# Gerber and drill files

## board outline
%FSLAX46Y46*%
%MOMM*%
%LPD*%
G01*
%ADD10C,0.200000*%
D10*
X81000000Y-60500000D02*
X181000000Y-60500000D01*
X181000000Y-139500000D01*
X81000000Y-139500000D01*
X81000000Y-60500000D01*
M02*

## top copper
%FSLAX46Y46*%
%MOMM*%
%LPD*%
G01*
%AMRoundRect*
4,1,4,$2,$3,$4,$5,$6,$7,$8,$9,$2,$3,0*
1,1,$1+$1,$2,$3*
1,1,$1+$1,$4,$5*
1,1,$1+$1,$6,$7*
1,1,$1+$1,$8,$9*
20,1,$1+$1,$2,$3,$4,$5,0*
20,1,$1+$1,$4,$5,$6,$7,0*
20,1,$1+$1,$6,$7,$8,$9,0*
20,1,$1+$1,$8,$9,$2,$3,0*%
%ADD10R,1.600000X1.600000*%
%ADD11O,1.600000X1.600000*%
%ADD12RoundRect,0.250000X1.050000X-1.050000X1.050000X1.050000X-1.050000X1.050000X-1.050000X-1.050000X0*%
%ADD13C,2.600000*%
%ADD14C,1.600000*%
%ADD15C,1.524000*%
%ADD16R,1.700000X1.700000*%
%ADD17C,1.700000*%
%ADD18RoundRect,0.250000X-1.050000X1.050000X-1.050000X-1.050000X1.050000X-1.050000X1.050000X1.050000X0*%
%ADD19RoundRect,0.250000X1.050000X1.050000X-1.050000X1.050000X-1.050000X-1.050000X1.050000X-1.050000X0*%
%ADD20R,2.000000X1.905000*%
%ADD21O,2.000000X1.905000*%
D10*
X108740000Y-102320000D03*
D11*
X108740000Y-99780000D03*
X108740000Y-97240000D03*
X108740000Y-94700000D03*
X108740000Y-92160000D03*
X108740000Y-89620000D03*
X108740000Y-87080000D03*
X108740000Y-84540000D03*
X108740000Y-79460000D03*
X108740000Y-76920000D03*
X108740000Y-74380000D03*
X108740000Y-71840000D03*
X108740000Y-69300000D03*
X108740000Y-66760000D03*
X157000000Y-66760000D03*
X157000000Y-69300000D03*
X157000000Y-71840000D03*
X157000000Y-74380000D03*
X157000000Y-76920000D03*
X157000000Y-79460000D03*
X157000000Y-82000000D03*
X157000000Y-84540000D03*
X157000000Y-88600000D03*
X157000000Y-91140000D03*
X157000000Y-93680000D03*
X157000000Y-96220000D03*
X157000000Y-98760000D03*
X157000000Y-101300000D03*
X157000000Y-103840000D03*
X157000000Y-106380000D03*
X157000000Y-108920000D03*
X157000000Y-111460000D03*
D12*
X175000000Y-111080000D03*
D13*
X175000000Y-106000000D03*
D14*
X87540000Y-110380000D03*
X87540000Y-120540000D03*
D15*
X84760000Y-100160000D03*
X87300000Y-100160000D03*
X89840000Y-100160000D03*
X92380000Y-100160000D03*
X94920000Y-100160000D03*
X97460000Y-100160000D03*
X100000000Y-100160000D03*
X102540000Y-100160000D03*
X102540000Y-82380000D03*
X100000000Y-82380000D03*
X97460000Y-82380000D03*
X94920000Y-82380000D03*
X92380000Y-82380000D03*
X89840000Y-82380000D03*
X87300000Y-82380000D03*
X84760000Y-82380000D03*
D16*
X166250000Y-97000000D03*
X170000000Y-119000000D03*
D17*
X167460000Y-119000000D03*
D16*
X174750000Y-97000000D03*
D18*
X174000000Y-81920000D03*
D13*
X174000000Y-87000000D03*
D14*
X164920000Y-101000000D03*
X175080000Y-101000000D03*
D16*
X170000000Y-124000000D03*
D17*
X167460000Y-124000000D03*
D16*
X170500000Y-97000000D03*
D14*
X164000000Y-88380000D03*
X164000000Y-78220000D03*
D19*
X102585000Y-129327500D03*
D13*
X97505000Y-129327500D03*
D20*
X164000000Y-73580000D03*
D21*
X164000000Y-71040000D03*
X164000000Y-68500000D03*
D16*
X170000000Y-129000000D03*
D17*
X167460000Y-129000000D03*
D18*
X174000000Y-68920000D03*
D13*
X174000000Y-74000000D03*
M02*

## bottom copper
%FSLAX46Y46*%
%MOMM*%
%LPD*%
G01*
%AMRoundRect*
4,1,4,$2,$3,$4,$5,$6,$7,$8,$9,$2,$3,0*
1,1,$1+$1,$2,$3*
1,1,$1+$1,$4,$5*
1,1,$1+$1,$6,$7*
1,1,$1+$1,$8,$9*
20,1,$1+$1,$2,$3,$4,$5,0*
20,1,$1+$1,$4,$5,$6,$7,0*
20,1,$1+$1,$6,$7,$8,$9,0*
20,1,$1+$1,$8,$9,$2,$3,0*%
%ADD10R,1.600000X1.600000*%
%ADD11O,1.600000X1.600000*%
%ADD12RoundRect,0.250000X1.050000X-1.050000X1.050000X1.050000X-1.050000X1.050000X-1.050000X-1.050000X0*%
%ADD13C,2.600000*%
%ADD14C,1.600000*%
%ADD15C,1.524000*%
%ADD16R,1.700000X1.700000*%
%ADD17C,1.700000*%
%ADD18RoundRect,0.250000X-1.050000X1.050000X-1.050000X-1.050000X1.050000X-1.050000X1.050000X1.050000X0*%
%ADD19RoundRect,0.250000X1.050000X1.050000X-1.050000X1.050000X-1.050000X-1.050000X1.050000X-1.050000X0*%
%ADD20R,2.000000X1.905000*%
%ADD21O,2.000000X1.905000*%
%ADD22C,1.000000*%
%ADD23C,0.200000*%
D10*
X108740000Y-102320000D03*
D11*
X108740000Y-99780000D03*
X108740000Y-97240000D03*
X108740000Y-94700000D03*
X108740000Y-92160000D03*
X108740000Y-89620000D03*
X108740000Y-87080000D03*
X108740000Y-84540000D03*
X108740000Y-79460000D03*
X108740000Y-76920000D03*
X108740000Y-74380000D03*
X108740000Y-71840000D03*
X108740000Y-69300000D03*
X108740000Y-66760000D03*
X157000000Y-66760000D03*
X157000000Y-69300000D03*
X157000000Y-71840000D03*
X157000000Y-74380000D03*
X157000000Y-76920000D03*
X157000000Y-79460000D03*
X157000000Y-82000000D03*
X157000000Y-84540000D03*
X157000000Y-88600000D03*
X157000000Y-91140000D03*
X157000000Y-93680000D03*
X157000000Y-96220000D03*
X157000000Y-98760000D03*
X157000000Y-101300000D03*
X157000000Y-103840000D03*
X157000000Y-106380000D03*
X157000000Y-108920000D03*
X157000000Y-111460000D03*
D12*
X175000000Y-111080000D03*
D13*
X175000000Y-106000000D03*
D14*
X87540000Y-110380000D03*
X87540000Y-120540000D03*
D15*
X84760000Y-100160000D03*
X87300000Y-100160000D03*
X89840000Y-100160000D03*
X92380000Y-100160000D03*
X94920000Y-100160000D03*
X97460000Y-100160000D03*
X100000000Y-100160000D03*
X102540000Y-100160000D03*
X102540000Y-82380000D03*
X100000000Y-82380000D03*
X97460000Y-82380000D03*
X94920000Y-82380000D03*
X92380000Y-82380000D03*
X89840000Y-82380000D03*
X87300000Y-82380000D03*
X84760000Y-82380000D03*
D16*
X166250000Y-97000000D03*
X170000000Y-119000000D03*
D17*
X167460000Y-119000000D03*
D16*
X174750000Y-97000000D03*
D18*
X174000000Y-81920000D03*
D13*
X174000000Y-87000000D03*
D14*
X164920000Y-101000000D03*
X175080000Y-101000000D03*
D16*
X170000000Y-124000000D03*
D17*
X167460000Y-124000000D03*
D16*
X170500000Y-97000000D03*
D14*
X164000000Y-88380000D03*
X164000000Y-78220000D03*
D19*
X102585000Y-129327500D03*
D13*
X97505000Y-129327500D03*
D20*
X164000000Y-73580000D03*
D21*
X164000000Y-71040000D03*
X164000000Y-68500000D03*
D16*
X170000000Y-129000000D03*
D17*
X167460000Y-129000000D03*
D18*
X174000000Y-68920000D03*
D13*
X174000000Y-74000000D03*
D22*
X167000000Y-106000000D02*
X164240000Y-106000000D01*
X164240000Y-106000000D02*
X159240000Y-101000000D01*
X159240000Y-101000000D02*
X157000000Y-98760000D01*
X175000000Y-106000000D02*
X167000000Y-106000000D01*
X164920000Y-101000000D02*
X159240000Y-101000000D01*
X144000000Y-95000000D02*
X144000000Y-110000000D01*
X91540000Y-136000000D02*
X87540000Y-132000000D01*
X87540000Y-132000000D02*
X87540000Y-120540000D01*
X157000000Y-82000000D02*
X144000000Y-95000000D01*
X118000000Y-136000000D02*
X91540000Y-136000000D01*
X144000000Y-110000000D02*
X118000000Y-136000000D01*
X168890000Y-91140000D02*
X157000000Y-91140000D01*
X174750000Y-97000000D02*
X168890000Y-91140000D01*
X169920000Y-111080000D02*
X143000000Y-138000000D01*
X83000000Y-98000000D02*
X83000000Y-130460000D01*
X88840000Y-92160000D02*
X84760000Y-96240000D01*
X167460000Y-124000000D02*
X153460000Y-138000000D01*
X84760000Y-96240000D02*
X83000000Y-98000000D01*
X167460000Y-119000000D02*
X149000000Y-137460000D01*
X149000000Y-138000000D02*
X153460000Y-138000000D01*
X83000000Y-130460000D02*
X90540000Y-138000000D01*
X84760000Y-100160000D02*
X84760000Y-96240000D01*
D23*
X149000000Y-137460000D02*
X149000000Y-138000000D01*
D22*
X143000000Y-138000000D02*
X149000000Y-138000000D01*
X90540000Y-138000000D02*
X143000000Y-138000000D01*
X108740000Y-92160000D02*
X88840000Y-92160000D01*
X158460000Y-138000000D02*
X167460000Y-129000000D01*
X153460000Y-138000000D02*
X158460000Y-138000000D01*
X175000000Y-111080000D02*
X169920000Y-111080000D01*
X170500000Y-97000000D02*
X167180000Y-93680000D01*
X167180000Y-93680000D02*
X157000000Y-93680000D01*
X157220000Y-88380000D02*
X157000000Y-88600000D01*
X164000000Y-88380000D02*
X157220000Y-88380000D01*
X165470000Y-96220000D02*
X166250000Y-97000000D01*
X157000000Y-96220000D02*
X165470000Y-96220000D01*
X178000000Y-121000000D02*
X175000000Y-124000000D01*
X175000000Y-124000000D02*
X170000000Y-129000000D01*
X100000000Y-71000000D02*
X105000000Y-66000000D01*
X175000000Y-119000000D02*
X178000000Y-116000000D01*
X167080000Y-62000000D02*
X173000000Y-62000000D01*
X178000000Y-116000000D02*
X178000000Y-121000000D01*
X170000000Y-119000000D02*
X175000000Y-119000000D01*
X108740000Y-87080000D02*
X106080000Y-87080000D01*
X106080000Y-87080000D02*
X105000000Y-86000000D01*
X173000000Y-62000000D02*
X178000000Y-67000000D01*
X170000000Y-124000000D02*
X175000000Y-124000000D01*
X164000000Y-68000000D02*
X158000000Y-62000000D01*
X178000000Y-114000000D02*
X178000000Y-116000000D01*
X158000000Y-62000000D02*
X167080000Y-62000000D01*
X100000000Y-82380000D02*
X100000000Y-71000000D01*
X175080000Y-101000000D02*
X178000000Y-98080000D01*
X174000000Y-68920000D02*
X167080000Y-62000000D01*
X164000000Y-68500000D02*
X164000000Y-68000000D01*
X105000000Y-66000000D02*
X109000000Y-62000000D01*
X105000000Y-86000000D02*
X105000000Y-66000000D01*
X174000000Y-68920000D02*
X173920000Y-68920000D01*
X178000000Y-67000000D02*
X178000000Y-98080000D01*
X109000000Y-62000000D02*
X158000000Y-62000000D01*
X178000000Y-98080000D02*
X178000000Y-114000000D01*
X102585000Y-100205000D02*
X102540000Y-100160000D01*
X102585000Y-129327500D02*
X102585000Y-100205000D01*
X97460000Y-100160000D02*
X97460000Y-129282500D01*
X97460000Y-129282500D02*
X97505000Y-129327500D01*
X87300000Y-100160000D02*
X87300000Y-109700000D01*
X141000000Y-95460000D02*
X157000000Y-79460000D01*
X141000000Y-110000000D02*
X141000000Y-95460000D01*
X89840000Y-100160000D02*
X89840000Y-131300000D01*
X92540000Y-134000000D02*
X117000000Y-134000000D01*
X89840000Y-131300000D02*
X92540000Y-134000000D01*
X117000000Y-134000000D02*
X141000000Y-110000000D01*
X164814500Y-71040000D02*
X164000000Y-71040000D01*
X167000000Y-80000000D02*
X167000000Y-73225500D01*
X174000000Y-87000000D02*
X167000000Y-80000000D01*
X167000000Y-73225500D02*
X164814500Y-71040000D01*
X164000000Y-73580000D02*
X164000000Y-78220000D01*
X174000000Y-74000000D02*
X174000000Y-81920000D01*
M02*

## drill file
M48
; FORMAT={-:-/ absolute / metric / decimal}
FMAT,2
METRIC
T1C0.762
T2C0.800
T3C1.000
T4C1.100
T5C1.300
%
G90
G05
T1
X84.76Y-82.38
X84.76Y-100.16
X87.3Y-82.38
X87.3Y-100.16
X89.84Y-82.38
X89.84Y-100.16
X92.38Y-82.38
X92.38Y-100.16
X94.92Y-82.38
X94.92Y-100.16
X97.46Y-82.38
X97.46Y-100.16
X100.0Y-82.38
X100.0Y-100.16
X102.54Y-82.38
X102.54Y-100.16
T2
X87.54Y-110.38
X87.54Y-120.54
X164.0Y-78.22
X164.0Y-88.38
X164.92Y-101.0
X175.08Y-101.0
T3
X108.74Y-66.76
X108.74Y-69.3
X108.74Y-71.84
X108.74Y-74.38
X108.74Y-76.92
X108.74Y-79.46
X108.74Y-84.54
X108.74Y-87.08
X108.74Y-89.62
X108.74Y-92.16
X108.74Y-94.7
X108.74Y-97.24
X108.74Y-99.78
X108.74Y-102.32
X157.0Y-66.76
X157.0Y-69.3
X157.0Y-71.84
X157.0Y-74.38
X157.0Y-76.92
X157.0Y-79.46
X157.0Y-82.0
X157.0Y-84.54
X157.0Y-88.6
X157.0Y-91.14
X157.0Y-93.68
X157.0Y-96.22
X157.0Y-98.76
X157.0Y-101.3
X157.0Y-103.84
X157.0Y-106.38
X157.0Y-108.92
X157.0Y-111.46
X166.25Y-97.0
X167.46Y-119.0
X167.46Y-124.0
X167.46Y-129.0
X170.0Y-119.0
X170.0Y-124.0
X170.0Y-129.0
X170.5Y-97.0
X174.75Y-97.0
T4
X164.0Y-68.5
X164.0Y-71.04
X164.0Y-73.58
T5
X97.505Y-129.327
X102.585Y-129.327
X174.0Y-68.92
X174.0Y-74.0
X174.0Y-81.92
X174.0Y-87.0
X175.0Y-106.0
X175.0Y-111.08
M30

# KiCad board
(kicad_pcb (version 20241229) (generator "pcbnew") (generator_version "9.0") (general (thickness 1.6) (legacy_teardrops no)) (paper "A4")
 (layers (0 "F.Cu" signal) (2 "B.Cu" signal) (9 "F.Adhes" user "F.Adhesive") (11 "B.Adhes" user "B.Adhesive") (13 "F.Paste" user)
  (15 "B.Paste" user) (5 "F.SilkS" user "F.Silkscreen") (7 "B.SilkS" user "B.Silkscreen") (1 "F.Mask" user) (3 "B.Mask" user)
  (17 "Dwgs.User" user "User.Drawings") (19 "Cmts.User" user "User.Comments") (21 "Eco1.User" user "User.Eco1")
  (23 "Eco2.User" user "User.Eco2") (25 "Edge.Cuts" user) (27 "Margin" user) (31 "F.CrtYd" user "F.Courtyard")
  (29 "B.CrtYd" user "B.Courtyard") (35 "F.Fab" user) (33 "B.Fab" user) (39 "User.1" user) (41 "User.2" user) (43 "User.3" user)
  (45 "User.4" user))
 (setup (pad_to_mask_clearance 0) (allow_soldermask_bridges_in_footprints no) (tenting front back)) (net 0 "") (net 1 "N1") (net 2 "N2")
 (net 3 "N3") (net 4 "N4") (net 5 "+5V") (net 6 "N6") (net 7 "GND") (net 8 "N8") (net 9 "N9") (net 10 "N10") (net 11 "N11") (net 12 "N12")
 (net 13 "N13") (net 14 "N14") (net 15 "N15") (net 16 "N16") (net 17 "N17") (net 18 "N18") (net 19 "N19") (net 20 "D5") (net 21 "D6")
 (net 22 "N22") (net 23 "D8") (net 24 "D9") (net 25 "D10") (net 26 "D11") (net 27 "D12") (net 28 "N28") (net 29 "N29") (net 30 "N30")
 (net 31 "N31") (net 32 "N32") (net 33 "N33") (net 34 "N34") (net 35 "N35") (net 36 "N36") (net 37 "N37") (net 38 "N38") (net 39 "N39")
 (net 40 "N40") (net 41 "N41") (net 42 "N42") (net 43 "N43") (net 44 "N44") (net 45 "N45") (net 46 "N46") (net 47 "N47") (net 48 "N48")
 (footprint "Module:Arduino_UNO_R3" (layer "F.Cu") (at 108.74 102.32 90)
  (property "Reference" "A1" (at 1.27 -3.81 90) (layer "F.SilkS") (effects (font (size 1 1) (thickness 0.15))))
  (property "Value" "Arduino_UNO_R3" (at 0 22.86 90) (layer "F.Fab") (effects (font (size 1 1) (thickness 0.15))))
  (pad "1" thru_hole rect (at 0 0 180) (size 1.6 1.6) (drill 1) (layers "*.Cu" "*.Mask") (remove_unused_layers no) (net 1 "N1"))
  (pad "2" thru_hole oval (at 2.54 0 180) (size 1.6 1.6) (drill 1) (layers "*.Cu" "*.Mask") (remove_unused_layers no) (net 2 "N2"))
  (pad "3" thru_hole oval (at 5.08 0 180) (size 1.6 1.6) (drill 1) (layers "*.Cu" "*.Mask") (remove_unused_layers no) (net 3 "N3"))
  (pad "4" thru_hole oval (at 7.62 0 180) (size 1.6 1.6) (drill 1) (layers "*.Cu" "*.Mask") (remove_unused_layers no) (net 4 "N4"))
  (pad "5" thru_hole oval (at 10.16 0 180) (size 1.6 1.6) (drill 1) (layers "*.Cu" "*.Mask") (remove_unused_layers no) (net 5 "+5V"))
  (pad "6" thru_hole oval (at 12.7 0 180) (size 1.6 1.6) (drill 1) (layers "*.Cu" "*.Mask") (remove_unused_layers no) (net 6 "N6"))
  (pad "7" thru_hole oval (at 15.24 0 180) (size 1.6 1.6) (drill 1) (layers "*.Cu" "*.Mask") (remove_unused_layers no) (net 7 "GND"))
  (pad "8" thru_hole oval (at 17.78 0 180) (size 1.6 1.6) (drill 1) (layers "*.Cu" "*.Mask") (remove_unused_layers no) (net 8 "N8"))
  (pad "9" thru_hole oval (at 22.86 0 180) (size 1.6 1.6) (drill 1) (layers "*.Cu" "*.Mask") (remove_unused_layers no) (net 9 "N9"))
  (pad "10" thru_hole oval (at 25.4 0 180) (size 1.6 1.6) (drill 1) (layers "*.Cu" "*.Mask") (remove_unused_layers no) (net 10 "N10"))
  (pad "11" thru_hole oval (at 27.94 0 180) (size 1.6 1.6) (drill 1) (layers "*.Cu" "*.Mask") (remove_unused_layers no) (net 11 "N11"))
  (pad "12" thru_hole oval (at 30.48 0 180) (size 1.6 1.6) (drill 1) (layers "*.Cu" "*.Mask") (remove_unused_layers no) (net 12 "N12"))
  (pad "13" thru_hole oval (at 33.02 0 180) (size 1.6 1.6) (drill 1) (layers "*.Cu" "*.Mask") (remove_unused_layers no) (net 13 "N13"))
  (pad "14" thru_hole oval (at 35.56 0 180) (size 1.6 1.6) (drill 1) (layers "*.Cu" "*.Mask") (remove_unused_layers no) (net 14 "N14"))
  (pad "15" thru_hole oval (at 35.56 48.26 180) (size 1.6 1.6) (drill 1) (layers "*.Cu" "*.Mask") (remove_unused_layers no) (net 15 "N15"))
  (pad "16" thru_hole oval (at 33.02 48.26 180) (size 1.6 1.6) (drill 1) (layers "*.Cu" "*.Mask") (remove_unused_layers no) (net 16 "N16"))
  (pad "17" thru_hole oval (at 30.48 48.26 180) (size 1.6 1.6) (drill 1) (layers "*.Cu" "*.Mask") (remove_unused_layers no) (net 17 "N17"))
  (pad "18" thru_hole oval (at 27.94 48.26 180) (size 1.6 1.6) (drill 1) (layers "*.Cu" "*.Mask") (remove_unused_layers no) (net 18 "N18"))
  (pad "19" thru_hole oval (at 25.4 48.26 180) (size 1.6 1.6) (drill 1) (layers "*.Cu" "*.Mask") (remove_unused_layers no) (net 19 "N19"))
  (pad "20" thru_hole oval (at 22.86 48.26 180) (size 1.6 1.6) (drill 1) (layers "*.Cu" "*.Mask") (remove_unused_layers no) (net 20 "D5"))
  (pad "21" thru_hole oval (at 20.32 48.26 180) (size 1.6 1.6) (drill 1) (layers "*.Cu" "*.Mask") (remove_unused_layers no) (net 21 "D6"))
  (pad "22" thru_hole oval (at 17.78 48.26 180) (size 1.6 1.6) (drill 1) (layers "*.Cu" "*.Mask") (remove_unused_layers no) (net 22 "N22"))
  (pad "23" thru_hole oval (at 13.72 48.26 180) (size 1.6 1.6) (drill 1) (layers "*.Cu" "*.Mask") (remove_unused_layers no) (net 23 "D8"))
  (pad "24" thru_hole oval (at 11.18 48.26 180) (size 1.6 1.6) (drill 1) (layers "*.Cu" "*.Mask") (remove_unused_layers no) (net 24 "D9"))
  (pad "25" thru_hole oval (at 8.64 48.26 180) (size 1.6 1.6) (drill 1) (layers "*.Cu" "*.Mask") (remove_unused_layers no) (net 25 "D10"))
  (pad "26" thru_hole oval (at 6.1 48.26 180) (size 1.6 1.6) (drill 1) (layers "*.Cu" "*.Mask") (remove_unused_layers no) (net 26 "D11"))
  (pad "27" thru_hole oval (at 3.56 48.26 180) (size 1.6 1.6) (drill 1) (layers "*.Cu" "*.Mask") (remove_unused_layers no) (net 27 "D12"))
  (pad "28" thru_hole oval (at 1.02 48.26 180) (size 1.6 1.6) (drill 1) (layers "*.Cu" "*.Mask") (remove_unused_layers no) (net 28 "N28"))
  (pad "29" thru_hole oval (at -1.52 48.26 180) (size 1.6 1.6) (drill 1) (layers "*.Cu" "*.Mask") (remove_unused_layers no) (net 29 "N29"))
  (pad "30" thru_hole oval (at -4.06 48.26 180) (size 1.6 1.6) (drill 1) (layers "*.Cu" "*.Mask") (remove_unused_layers no) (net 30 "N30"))
  (pad "31" thru_hole oval (at -6.6 48.26 180) (size 1.6 1.6) (drill 1) (layers "*.Cu" "*.Mask") (remove_unused_layers no) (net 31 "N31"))
  (pad "32" thru_hole oval (at -9.14 48.26 180) (size 1.6 1.6) (drill 1) (layers "*.Cu" "*.Mask") (remove_unused_layers no) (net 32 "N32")))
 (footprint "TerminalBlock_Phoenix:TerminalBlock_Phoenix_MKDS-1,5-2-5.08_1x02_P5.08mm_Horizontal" (layer "F.Cu") (at 175 111.08 90)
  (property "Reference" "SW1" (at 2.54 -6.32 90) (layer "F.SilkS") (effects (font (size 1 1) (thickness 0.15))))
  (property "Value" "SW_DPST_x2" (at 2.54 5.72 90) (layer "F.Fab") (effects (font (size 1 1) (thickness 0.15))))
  (pad "1" thru_hole roundrect (at 0 0 90) (size 2.6 2.6) (drill 1.3) (layers "*.Cu" "*.Mask") (remove_unused_layers no)
   (roundrect_rratio 0.096154) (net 5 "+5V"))
  (pad "2" thru_hole circle (at 5.08 0 90) (size 2.6 2.6) (drill 1.3) (layers "*.Cu" "*.Mask") (remove_unused_layers no) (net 27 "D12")))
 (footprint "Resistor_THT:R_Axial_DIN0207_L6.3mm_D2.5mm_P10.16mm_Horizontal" (layer "F.Cu") (at 87.54 110.38 -90)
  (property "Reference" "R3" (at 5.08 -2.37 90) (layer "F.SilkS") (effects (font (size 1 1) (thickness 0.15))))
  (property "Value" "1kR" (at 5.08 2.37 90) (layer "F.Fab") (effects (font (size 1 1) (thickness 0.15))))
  (pad "1" thru_hole circle (at 0 0 270) (size 1.6 1.6) (drill 0.8) (layers "*.Cu" "*.Mask") (remove_unused_layers no) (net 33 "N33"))
  (pad "2" thru_hole circle (at 10.16 0 270) (size 1.6 1.6) (drill 0.8) (layers "*.Cu" "*.Mask") (remove_unused_layers no) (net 21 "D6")))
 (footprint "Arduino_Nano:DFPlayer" (layer "F.Cu") (at 84.76 92.54 90)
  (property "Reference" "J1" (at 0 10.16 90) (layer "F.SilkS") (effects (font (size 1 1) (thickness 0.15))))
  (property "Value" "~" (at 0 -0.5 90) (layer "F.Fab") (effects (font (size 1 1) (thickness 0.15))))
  (pad "1" thru_hole circle (at -7.62 0 90) (size 1.524 1.524) (drill 0.762) (layers "*.Cu" "*.Mask") (remove_unused_layers no)
   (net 5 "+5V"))
  (pad "2" thru_hole circle (at -7.62 2.54 90) (size 1.524 1.524) (drill 0.762) (layers "*.Cu" "*.Mask") (remove_unused_layers no)
   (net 33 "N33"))
  (pad "3" thru_hole circle (at -7.62 5.08 90) (size 1.524 1.524) (drill 0.762) (layers "*.Cu" "*.Mask") (remove_unused_layers no)
   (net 20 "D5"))
  (pad "4" thru_hole circle (at -7.62 7.62 90) (size 1.524 1.524) (drill 0.762) (layers "*.Cu" "*.Mask") (remove_unused_layers no)
   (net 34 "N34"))
  (pad "5" thru_hole circle (at -7.62 10.16 90) (size 1.524 1.524) (drill 0.762) (layers "*.Cu" "*.Mask") (remove_unused_layers no)
   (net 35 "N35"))
  (pad "6" thru_hole circle (at -7.62 12.7 90) (size 1.524 1.524) (drill 0.762) (layers "*.Cu" "*.Mask") (remove_unused_layers no)
   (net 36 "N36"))
  (pad "7" thru_hole circle (at -7.62 15.24 90) (size 1.524 1.524) (drill 0.762) (layers "*.Cu" "*.Mask") (remove_unused_layers no)
   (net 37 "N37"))
  (pad "8" thru_hole circle (at -7.62 17.78 90) (size 1.524 1.524) (drill 0.762) (layers "*.Cu" "*.Mask") (remove_unused_layers no)
   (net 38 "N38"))
  (pad "9" thru_hole circle (at 10.16 17.78 90) (size 1.524 1.524) (drill 0.762) (layers "*.Cu" "*.Mask") (remove_unused_layers no)
   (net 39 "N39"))
  (pad "10" thru_hole circle (at 10.16 15.24 90) (size 1.524 1.524) (drill 0.762) (layers "*.Cu" "*.Mask") (remove_unused_layers no)
   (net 7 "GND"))
  (pad "11" thru_hole circle (at 10.16 12.7 90) (size 1.524 1.524) (drill 0.762) (layers "*.Cu" "*.Mask") (remove_unused_layers no)
   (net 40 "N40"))
  (pad "12" thru_hole circle (at 10.16 10.16 90) (size 1.524 1.524) (drill 0.762) (layers "*.Cu" "*.Mask") (remove_unused_layers no)
   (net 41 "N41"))
  (pad "13" thru_hole circle (at 10.16 7.62 90) (size 1.524 1.524) (drill 0.762) (layers "*.Cu" "*.Mask") (remove_unused_layers no)
   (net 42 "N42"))
  (pad "14" thru_hole circle (at 10.16 5.08 90) (size 1.524 1.524) (drill 0.762) (layers "*.Cu" "*.Mask") (remove_unused_layers no)
   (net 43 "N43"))
  (pad "15" thru_hole circle (at 10.16 2.54 90) (size 1.524 1.524) (drill 0.762) (layers "*.Cu" "*.Mask") (remove_unused_layers no)
   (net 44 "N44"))
  (pad "16" thru_hole circle (at 10.16 0 90) (size 1.524 1.524) (drill 0.762) (layers "*.Cu" "*.Mask") (remove_unused_layers no)
   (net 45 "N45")))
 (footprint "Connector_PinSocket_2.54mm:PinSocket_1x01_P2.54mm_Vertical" (layer "F.Cu") (at 166.25 97 -90)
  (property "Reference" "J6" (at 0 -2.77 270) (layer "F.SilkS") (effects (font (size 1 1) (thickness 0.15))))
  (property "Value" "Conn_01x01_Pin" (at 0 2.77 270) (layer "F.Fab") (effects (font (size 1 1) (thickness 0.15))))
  (pad "1" thru_hole rect (at 0 0 270) (size 1.7 1.7) (drill 1) (layers "*.Cu" "*.Mask") (remove_unused_layers no) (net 26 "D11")))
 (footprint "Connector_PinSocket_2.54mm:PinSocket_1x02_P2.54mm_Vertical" (layer "F.Cu") (at 170 119 -90)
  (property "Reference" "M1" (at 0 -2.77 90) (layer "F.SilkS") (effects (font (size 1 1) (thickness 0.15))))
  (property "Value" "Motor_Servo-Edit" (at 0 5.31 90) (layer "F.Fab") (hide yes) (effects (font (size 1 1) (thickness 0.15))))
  (pad "1" thru_hole rect (at 0 0 270) (size 1.7 1.7) (drill 1) (layers "*.Cu" "*.Mask") (remove_unused_layers no) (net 7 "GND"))
  (pad "2" thru_hole circle (at 0 2.54 270) (size 1.7 1.7) (drill 1) (layers "*.Cu" "*.Mask") (remove_unused_layers no) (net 5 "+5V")))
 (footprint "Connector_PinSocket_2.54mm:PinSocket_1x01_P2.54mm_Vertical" (layer "F.Cu") (at 174.75 97 -90)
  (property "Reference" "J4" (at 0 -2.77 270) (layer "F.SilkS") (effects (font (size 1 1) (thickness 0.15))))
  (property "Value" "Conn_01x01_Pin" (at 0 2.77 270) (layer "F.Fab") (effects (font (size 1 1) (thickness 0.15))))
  (pad "1" thru_hole rect (at 0 0 270) (size 1.7 1.7) (drill 1) (layers "*.Cu" "*.Mask") (remove_unused_layers no) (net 24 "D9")))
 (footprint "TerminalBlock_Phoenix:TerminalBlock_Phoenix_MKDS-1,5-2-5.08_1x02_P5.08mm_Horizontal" (layer "F.Cu") (at 174 81.92 -90)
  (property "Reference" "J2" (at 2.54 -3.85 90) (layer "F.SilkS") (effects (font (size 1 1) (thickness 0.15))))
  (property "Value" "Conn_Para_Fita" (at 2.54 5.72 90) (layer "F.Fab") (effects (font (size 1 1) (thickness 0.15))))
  (pad "1" thru_hole roundrect (at 0 0 270) (size 2.6 2.6) (drill 1.3) (layers "*.Cu" "*.Mask") (remove_unused_layers no)
   (roundrect_rratio 0.096154) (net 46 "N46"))
  (pad "2" thru_hole circle (at 5.08 0 270) (size 2.6 2.6) (drill 1.3) (layers "*.Cu" "*.Mask") (remove_unused_layers no) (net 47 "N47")))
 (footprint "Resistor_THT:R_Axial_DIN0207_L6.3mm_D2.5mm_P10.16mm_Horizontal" (layer "F.Cu") (at 164.92 101)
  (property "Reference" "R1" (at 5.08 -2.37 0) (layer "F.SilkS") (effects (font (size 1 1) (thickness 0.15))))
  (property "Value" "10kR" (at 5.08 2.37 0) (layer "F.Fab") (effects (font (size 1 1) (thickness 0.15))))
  (pad "1" thru_hole circle (at 0 0) (size 1.6 1.6) (drill 0.8) (layers "*.Cu" "*.Mask") (remove_unused_layers no) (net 27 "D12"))
  (pad "2" thru_hole circle (at 10.16 0) (size 1.6 1.6) (drill 0.8) (layers "*.Cu" "*.Mask") (remove_unused_layers no) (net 7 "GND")))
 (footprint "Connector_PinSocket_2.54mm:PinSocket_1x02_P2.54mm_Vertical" (layer "F.Cu") (at 170 124 -90)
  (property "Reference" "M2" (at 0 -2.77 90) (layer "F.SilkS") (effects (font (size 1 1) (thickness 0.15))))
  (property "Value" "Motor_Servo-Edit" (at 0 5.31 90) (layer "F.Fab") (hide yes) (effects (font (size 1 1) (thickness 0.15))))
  (pad "1" thru_hole rect (at 0 0 270) (size 1.7 1.7) (drill 1) (layers "*.Cu" "*.Mask") (remove_unused_layers no) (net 7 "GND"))
  (pad "2" thru_hole circle (at 0 2.54 270) (size 1.7 1.7) (drill 1) (layers "*.Cu" "*.Mask") (remove_unused_layers no) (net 5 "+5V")))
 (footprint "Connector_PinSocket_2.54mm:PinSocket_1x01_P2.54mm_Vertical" (layer "F.Cu") (at 170.5 97 -90)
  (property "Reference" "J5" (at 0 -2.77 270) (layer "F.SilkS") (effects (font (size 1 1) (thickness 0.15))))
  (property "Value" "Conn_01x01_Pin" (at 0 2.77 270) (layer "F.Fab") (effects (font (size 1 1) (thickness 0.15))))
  (pad "1" thru_hole rect (at 0 0 270) (size 1.7 1.7) (drill 1) (layers "*.Cu" "*.Mask") (remove_unused_layers no) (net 25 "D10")))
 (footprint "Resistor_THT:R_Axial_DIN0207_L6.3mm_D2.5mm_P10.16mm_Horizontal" (layer "F.Cu") (at 164 88.38 90)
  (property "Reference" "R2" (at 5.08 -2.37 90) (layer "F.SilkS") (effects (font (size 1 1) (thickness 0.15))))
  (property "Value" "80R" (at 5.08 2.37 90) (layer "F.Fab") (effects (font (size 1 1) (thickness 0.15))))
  (pad "1" thru_hole circle (at 0 0 90) (size 1.6 1.6) (drill 0.8) (layers "*.Cu" "*.Mask") (remove_unused_layers no) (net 23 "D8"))
  (pad "2" thru_hole circle (at 10.16 0 90) (size 1.6 1.6) (drill 0.8) (layers "*.Cu" "*.Mask") (remove_unused_layers no) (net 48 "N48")))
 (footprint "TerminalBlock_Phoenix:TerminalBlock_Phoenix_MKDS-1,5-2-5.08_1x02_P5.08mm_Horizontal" (layer "F.Cu") (at 102.585 129.3275 180)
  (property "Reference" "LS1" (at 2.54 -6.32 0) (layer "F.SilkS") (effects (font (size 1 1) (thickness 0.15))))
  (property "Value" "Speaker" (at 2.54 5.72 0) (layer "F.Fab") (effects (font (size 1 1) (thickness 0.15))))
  (pad "1" thru_hole roundrect (at 0 0 180) (size 2.6 2.6) (drill 1.3) (layers "*.Cu" "*.Mask") (remove_unused_layers no)
   (roundrect_rratio 0.096154) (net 38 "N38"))
  (pad "2" thru_hole circle (at 5.08 0 180) (size 2.6 2.6) (drill 1.3) (layers "*.Cu" "*.Mask") (remove_unused_layers no) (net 36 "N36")))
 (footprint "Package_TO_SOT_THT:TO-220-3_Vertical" (layer "F.Cu") (at 164 73.58 90)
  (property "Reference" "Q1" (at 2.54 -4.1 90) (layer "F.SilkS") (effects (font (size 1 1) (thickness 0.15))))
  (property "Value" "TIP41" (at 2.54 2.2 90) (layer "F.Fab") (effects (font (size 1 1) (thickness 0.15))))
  (pad "1" thru_hole rect (at 0 0 90) (size 1.905 2) (drill 1.1) (layers "*.Cu" "*.Mask") (remove_unused_layers no) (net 48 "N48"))
  (pad "2" thru_hole oval (at 2.54 0 90) (size 1.905 2) (drill 1.1) (layers "*.Cu" "*.Mask") (remove_unused_layers no) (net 47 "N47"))
  (pad "3" thru_hole oval (at 5.08 0 90) (size 1.905 2) (drill 1.1) (layers "*.Cu" "*.Mask") (remove_unused_layers no) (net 7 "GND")))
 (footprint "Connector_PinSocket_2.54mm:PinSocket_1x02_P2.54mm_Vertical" (layer "F.Cu") (at 170 129 -90)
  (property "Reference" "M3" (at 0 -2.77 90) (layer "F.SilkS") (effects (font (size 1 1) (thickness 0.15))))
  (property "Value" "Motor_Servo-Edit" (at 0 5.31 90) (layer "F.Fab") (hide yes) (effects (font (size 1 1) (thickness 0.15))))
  (pad "1" thru_hole rect (at 0 0 270) (size 1.7 1.7) (drill 1) (layers "*.Cu" "*.Mask") (remove_unused_layers no) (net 7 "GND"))
  (pad "2" thru_hole circle (at 0 2.54 270) (size 1.7 1.7) (drill 1) (layers "*.Cu" "*.Mask") (remove_unused_layers no) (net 5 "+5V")))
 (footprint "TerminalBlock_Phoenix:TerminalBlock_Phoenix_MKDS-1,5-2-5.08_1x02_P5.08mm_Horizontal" (layer "F.Cu") (at 174 68.92 -90)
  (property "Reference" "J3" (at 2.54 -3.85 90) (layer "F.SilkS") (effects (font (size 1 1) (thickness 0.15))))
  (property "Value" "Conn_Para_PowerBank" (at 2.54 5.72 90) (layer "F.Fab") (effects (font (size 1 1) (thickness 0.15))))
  (pad "1" thru_hole roundrect (at 0 0 270) (size 2.6 2.6) (drill 1.3) (layers "*.Cu" "*.Mask") (remove_unused_layers no)
   (roundrect_rratio 0.096154) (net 7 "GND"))
  (pad "2" thru_hole circle (at 5.08 0 270) (size 2.6 2.6) (drill 1.3) (layers "*.Cu" "*.Mask") (remove_unused_layers no) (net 46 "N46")))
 (gr_rect (start 81 60.5) (end 181 139.5) (stroke (width 0.2) (type solid)) (fill no) (layer "Edge.Cuts"))
 (segment (start 167 106) (end 164.24 106) (width 1) (layer "B.Cu") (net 27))
 (segment (start 164.24 106) (end 159.24 101) (width 1) (layer "B.Cu") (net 27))
 (segment (start 159.24 101) (end 157 98.76) (width 1) (layer "B.Cu") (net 27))
 (segment (start 175 106) (end 167 106) (width 1) (layer "B.Cu") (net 27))
 (segment (start 164.92 101) (end 159.24 101) (width 1) (layer "B.Cu") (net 27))
 (segment (start 144 95) (end 144 110) (width 1) (layer "B.Cu") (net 21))
 (segment (start 91.54 136) (end 87.54 132) (width 1) (layer "B.Cu") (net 21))
 (segment (start 87.54 132) (end 87.54 120.54) (width 1) (layer "B.Cu") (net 21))
 (segment (start 157 82) (end 144 95) (width 1) (layer "B.Cu") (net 21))
 (segment (start 118 136) (end 91.54 136) (width 1) (layer "B.Cu") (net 21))
 (segment (start 144 110) (end 118 136) (width 1) (layer "B.Cu") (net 21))
 (segment (start 168.89 91.14) (end 157 91.14) (width 1) (layer "B.Cu") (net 24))
 (segment (start 174.75 97) (end 168.89 91.14) (width 1) (layer "B.Cu") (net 24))
 (segment (start 169.92 111.08) (end 143 138) (width 1) (layer "B.Cu") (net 5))
 (segment (start 83 98) (end 83 130.46) (width 1) (layer "B.Cu") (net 5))
 (segment (start 88.84 92.16) (end 84.76 96.24) (width 1) (layer "B.Cu") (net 5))
 (segment (start 167.46 124) (end 153.46 138) (width 1) (layer "B.Cu") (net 5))
 (segment (start 84.76 96.24) (end 83 98) (width 1) (layer "B.Cu") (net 5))
 (segment (start 167.46 119) (end 149 137.46) (width 1) (layer "B.Cu") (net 5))
 (segment (start 149 138) (end 153.46 138) (width 1) (layer "B.Cu") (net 5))
 (segment (start 83 130.46) (end 90.54 138) (width 1) (layer "B.Cu") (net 5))
 (segment (start 84.76 100.16) (end 84.76 96.24) (width 1) (layer "B.Cu") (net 5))
 (segment (start 149 137.46) (end 149 138) (width 0.2) (layer "B.Cu") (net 5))
 (segment (start 143 138) (end 149 138) (width 1) (layer "B.Cu") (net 5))
 (segment (start 90.54 138) (end 143 138) (width 1) (layer "B.Cu") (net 5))
 (segment (start 108.74 92.16) (end 88.84 92.16) (width 1) (layer "B.Cu") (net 5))
 (segment (start 158.46 138) (end 167.46 129) (width 1) (layer "B.Cu") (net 5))
 (segment (start 153.46 138) (end 158.46 138) (width 1) (layer "B.Cu") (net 5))
 (segment (start 175 111.08) (end 169.92 111.08) (width 1) (layer "B.Cu") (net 5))
 (segment (start 170.5 97) (end 167.18 93.68) (width 1) (layer "B.Cu") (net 25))
 (segment (start 167.18 93.68) (end 157 93.68) (width 1) (layer "B.Cu") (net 25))
 (segment (start 157.22 88.38) (end 157 88.6) (width 1) (layer "B.Cu") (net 23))
 (segment (start 164 88.38) (end 157.22 88.38) (width 1) (layer "B.Cu") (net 23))
 (segment (start 165.47 96.22) (end 166.25 97) (width 1) (layer "B.Cu") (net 26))
 (segment (start 157 96.22) (end 165.47 96.22) (width 1) (layer "B.Cu") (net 26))
 (segment (start 178 121) (end 175 124) (width 1) (layer "B.Cu") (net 7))
 (segment (start 175 124) (end 170 129) (width 1) (layer "B.Cu") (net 7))
 (segment (start 100 71) (end 105 66) (width 1) (layer "B.Cu") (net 7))
 (segment (start 175 119) (end 178 116) (width 1) (layer "B.Cu") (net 7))
 (segment (start 167.08 62) (end 173 62) (width 1) (layer "B.Cu") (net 7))
 (segment (start 178 116) (end 178 121) (width 1) (layer "B.Cu") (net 7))
 (segment (start 170 119) (end 175 119) (width 1) (layer "B.Cu") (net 7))
 (segment (start 108.74 87.08) (end 106.08 87.08) (width 1) (layer "B.Cu") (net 7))
 (segment (start 106.08 87.08) (end 105 86) (width 1) (layer "B.Cu") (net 7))
 (segment (start 173 62) (end 178 67) (width 1) (layer "B.Cu") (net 7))
 (segment (start 170 124) (end 175 124) (width 1) (layer "B.Cu") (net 7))
 (segment (start 164 68) (end 158 62) (width 1) (layer "B.Cu") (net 7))
 (segment (start 178 114) (end 178 116) (width 1) (layer "B.Cu") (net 7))
 (segment (start 158 62) (end 167.08 62) (width 1) (layer "B.Cu") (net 7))
 (segment (start 100 82.38) (end 100 71) (width 1) (layer "B.Cu") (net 7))
 (segment (start 175.08 101) (end 178 98.08) (width 1) (layer "B.Cu") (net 7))
 (segment (start 174 68.92) (end 167.08 62) (width 1) (layer "B.Cu") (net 7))
 (segment (start 164 68.5) (end 164 68) (width 1) (layer "B.Cu") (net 7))
 (segment (start 105 66) (end 109 62) (width 1) (layer "B.Cu") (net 7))
 (segment (start 105 86) (end 105 66) (width 1) (layer "B.Cu") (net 7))
 (segment (start 174 68.92) (end 173.92 68.92) (width 1) (layer "B.Cu") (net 7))
 (segment (start 178 67) (end 178 98.08) (width 1) (layer "B.Cu") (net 7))
 (segment (start 109 62) (end 158 62) (width 1) (layer "B.Cu") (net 7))
 (segment (start 178 98.08) (end 178 114) (width 1) (layer "B.Cu") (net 7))
 (segment (start 102.585 100.205) (end 102.54 100.16) (width 1) (layer "B.Cu") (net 38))
 (segment (start 102.585 129.3275) (end 102.585 100.205) (width 1) (layer "B.Cu") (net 38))
 (segment (start 97.46 100.16) (end 97.46 129.2825) (width 1) (layer "B.Cu") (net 36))
 (segment (start 97.46 129.2825) (end 97.505 129.3275) (width 1) (layer "B.Cu") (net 36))
 (segment (start 87.3 100.16) (end 87.3 109.7) (width 1) (layer "B.Cu") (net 33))
 (segment (start 141 95.46) (end 157 79.46) (width 1) (layer "B.Cu") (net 20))
 (segment (start 141 110) (end 141 95.46) (width 1) (layer "B.Cu") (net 20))
 (segment (start 89.84 100.16) (end 89.84 131.3) (width 1) (layer "B.Cu") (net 20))
 (segment (start 92.54 134) (end 117 134) (width 1) (layer "B.Cu") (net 20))
 (segment (start 89.84 131.3) (end 92.54 134) (width 1) (layer "B.Cu") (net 20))
 (segment (start 117 134) (end 141 110) (width 1) (layer "B.Cu") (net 20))
 (segment (start 164.8145 71.04) (end 164 71.04) (width 1) (layer "B.Cu") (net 47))
 (segment (start 167 80) (end 167 73.2255) (width 1) (layer "B.Cu") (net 47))
 (segment (start 174 87) (end 167 80) (width 1) (layer "B.Cu") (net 47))
 (segment (start 167 73.2255) (end 164.8145 71.04) (width 1) (layer "B.Cu") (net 47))
 (segment (start 164 73.58) (end 164 78.22) (width 1) (layer "B.Cu") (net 48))
 (segment (start 174 74) (end 174 81.92) (width 1) (layer "B.Cu") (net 46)))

